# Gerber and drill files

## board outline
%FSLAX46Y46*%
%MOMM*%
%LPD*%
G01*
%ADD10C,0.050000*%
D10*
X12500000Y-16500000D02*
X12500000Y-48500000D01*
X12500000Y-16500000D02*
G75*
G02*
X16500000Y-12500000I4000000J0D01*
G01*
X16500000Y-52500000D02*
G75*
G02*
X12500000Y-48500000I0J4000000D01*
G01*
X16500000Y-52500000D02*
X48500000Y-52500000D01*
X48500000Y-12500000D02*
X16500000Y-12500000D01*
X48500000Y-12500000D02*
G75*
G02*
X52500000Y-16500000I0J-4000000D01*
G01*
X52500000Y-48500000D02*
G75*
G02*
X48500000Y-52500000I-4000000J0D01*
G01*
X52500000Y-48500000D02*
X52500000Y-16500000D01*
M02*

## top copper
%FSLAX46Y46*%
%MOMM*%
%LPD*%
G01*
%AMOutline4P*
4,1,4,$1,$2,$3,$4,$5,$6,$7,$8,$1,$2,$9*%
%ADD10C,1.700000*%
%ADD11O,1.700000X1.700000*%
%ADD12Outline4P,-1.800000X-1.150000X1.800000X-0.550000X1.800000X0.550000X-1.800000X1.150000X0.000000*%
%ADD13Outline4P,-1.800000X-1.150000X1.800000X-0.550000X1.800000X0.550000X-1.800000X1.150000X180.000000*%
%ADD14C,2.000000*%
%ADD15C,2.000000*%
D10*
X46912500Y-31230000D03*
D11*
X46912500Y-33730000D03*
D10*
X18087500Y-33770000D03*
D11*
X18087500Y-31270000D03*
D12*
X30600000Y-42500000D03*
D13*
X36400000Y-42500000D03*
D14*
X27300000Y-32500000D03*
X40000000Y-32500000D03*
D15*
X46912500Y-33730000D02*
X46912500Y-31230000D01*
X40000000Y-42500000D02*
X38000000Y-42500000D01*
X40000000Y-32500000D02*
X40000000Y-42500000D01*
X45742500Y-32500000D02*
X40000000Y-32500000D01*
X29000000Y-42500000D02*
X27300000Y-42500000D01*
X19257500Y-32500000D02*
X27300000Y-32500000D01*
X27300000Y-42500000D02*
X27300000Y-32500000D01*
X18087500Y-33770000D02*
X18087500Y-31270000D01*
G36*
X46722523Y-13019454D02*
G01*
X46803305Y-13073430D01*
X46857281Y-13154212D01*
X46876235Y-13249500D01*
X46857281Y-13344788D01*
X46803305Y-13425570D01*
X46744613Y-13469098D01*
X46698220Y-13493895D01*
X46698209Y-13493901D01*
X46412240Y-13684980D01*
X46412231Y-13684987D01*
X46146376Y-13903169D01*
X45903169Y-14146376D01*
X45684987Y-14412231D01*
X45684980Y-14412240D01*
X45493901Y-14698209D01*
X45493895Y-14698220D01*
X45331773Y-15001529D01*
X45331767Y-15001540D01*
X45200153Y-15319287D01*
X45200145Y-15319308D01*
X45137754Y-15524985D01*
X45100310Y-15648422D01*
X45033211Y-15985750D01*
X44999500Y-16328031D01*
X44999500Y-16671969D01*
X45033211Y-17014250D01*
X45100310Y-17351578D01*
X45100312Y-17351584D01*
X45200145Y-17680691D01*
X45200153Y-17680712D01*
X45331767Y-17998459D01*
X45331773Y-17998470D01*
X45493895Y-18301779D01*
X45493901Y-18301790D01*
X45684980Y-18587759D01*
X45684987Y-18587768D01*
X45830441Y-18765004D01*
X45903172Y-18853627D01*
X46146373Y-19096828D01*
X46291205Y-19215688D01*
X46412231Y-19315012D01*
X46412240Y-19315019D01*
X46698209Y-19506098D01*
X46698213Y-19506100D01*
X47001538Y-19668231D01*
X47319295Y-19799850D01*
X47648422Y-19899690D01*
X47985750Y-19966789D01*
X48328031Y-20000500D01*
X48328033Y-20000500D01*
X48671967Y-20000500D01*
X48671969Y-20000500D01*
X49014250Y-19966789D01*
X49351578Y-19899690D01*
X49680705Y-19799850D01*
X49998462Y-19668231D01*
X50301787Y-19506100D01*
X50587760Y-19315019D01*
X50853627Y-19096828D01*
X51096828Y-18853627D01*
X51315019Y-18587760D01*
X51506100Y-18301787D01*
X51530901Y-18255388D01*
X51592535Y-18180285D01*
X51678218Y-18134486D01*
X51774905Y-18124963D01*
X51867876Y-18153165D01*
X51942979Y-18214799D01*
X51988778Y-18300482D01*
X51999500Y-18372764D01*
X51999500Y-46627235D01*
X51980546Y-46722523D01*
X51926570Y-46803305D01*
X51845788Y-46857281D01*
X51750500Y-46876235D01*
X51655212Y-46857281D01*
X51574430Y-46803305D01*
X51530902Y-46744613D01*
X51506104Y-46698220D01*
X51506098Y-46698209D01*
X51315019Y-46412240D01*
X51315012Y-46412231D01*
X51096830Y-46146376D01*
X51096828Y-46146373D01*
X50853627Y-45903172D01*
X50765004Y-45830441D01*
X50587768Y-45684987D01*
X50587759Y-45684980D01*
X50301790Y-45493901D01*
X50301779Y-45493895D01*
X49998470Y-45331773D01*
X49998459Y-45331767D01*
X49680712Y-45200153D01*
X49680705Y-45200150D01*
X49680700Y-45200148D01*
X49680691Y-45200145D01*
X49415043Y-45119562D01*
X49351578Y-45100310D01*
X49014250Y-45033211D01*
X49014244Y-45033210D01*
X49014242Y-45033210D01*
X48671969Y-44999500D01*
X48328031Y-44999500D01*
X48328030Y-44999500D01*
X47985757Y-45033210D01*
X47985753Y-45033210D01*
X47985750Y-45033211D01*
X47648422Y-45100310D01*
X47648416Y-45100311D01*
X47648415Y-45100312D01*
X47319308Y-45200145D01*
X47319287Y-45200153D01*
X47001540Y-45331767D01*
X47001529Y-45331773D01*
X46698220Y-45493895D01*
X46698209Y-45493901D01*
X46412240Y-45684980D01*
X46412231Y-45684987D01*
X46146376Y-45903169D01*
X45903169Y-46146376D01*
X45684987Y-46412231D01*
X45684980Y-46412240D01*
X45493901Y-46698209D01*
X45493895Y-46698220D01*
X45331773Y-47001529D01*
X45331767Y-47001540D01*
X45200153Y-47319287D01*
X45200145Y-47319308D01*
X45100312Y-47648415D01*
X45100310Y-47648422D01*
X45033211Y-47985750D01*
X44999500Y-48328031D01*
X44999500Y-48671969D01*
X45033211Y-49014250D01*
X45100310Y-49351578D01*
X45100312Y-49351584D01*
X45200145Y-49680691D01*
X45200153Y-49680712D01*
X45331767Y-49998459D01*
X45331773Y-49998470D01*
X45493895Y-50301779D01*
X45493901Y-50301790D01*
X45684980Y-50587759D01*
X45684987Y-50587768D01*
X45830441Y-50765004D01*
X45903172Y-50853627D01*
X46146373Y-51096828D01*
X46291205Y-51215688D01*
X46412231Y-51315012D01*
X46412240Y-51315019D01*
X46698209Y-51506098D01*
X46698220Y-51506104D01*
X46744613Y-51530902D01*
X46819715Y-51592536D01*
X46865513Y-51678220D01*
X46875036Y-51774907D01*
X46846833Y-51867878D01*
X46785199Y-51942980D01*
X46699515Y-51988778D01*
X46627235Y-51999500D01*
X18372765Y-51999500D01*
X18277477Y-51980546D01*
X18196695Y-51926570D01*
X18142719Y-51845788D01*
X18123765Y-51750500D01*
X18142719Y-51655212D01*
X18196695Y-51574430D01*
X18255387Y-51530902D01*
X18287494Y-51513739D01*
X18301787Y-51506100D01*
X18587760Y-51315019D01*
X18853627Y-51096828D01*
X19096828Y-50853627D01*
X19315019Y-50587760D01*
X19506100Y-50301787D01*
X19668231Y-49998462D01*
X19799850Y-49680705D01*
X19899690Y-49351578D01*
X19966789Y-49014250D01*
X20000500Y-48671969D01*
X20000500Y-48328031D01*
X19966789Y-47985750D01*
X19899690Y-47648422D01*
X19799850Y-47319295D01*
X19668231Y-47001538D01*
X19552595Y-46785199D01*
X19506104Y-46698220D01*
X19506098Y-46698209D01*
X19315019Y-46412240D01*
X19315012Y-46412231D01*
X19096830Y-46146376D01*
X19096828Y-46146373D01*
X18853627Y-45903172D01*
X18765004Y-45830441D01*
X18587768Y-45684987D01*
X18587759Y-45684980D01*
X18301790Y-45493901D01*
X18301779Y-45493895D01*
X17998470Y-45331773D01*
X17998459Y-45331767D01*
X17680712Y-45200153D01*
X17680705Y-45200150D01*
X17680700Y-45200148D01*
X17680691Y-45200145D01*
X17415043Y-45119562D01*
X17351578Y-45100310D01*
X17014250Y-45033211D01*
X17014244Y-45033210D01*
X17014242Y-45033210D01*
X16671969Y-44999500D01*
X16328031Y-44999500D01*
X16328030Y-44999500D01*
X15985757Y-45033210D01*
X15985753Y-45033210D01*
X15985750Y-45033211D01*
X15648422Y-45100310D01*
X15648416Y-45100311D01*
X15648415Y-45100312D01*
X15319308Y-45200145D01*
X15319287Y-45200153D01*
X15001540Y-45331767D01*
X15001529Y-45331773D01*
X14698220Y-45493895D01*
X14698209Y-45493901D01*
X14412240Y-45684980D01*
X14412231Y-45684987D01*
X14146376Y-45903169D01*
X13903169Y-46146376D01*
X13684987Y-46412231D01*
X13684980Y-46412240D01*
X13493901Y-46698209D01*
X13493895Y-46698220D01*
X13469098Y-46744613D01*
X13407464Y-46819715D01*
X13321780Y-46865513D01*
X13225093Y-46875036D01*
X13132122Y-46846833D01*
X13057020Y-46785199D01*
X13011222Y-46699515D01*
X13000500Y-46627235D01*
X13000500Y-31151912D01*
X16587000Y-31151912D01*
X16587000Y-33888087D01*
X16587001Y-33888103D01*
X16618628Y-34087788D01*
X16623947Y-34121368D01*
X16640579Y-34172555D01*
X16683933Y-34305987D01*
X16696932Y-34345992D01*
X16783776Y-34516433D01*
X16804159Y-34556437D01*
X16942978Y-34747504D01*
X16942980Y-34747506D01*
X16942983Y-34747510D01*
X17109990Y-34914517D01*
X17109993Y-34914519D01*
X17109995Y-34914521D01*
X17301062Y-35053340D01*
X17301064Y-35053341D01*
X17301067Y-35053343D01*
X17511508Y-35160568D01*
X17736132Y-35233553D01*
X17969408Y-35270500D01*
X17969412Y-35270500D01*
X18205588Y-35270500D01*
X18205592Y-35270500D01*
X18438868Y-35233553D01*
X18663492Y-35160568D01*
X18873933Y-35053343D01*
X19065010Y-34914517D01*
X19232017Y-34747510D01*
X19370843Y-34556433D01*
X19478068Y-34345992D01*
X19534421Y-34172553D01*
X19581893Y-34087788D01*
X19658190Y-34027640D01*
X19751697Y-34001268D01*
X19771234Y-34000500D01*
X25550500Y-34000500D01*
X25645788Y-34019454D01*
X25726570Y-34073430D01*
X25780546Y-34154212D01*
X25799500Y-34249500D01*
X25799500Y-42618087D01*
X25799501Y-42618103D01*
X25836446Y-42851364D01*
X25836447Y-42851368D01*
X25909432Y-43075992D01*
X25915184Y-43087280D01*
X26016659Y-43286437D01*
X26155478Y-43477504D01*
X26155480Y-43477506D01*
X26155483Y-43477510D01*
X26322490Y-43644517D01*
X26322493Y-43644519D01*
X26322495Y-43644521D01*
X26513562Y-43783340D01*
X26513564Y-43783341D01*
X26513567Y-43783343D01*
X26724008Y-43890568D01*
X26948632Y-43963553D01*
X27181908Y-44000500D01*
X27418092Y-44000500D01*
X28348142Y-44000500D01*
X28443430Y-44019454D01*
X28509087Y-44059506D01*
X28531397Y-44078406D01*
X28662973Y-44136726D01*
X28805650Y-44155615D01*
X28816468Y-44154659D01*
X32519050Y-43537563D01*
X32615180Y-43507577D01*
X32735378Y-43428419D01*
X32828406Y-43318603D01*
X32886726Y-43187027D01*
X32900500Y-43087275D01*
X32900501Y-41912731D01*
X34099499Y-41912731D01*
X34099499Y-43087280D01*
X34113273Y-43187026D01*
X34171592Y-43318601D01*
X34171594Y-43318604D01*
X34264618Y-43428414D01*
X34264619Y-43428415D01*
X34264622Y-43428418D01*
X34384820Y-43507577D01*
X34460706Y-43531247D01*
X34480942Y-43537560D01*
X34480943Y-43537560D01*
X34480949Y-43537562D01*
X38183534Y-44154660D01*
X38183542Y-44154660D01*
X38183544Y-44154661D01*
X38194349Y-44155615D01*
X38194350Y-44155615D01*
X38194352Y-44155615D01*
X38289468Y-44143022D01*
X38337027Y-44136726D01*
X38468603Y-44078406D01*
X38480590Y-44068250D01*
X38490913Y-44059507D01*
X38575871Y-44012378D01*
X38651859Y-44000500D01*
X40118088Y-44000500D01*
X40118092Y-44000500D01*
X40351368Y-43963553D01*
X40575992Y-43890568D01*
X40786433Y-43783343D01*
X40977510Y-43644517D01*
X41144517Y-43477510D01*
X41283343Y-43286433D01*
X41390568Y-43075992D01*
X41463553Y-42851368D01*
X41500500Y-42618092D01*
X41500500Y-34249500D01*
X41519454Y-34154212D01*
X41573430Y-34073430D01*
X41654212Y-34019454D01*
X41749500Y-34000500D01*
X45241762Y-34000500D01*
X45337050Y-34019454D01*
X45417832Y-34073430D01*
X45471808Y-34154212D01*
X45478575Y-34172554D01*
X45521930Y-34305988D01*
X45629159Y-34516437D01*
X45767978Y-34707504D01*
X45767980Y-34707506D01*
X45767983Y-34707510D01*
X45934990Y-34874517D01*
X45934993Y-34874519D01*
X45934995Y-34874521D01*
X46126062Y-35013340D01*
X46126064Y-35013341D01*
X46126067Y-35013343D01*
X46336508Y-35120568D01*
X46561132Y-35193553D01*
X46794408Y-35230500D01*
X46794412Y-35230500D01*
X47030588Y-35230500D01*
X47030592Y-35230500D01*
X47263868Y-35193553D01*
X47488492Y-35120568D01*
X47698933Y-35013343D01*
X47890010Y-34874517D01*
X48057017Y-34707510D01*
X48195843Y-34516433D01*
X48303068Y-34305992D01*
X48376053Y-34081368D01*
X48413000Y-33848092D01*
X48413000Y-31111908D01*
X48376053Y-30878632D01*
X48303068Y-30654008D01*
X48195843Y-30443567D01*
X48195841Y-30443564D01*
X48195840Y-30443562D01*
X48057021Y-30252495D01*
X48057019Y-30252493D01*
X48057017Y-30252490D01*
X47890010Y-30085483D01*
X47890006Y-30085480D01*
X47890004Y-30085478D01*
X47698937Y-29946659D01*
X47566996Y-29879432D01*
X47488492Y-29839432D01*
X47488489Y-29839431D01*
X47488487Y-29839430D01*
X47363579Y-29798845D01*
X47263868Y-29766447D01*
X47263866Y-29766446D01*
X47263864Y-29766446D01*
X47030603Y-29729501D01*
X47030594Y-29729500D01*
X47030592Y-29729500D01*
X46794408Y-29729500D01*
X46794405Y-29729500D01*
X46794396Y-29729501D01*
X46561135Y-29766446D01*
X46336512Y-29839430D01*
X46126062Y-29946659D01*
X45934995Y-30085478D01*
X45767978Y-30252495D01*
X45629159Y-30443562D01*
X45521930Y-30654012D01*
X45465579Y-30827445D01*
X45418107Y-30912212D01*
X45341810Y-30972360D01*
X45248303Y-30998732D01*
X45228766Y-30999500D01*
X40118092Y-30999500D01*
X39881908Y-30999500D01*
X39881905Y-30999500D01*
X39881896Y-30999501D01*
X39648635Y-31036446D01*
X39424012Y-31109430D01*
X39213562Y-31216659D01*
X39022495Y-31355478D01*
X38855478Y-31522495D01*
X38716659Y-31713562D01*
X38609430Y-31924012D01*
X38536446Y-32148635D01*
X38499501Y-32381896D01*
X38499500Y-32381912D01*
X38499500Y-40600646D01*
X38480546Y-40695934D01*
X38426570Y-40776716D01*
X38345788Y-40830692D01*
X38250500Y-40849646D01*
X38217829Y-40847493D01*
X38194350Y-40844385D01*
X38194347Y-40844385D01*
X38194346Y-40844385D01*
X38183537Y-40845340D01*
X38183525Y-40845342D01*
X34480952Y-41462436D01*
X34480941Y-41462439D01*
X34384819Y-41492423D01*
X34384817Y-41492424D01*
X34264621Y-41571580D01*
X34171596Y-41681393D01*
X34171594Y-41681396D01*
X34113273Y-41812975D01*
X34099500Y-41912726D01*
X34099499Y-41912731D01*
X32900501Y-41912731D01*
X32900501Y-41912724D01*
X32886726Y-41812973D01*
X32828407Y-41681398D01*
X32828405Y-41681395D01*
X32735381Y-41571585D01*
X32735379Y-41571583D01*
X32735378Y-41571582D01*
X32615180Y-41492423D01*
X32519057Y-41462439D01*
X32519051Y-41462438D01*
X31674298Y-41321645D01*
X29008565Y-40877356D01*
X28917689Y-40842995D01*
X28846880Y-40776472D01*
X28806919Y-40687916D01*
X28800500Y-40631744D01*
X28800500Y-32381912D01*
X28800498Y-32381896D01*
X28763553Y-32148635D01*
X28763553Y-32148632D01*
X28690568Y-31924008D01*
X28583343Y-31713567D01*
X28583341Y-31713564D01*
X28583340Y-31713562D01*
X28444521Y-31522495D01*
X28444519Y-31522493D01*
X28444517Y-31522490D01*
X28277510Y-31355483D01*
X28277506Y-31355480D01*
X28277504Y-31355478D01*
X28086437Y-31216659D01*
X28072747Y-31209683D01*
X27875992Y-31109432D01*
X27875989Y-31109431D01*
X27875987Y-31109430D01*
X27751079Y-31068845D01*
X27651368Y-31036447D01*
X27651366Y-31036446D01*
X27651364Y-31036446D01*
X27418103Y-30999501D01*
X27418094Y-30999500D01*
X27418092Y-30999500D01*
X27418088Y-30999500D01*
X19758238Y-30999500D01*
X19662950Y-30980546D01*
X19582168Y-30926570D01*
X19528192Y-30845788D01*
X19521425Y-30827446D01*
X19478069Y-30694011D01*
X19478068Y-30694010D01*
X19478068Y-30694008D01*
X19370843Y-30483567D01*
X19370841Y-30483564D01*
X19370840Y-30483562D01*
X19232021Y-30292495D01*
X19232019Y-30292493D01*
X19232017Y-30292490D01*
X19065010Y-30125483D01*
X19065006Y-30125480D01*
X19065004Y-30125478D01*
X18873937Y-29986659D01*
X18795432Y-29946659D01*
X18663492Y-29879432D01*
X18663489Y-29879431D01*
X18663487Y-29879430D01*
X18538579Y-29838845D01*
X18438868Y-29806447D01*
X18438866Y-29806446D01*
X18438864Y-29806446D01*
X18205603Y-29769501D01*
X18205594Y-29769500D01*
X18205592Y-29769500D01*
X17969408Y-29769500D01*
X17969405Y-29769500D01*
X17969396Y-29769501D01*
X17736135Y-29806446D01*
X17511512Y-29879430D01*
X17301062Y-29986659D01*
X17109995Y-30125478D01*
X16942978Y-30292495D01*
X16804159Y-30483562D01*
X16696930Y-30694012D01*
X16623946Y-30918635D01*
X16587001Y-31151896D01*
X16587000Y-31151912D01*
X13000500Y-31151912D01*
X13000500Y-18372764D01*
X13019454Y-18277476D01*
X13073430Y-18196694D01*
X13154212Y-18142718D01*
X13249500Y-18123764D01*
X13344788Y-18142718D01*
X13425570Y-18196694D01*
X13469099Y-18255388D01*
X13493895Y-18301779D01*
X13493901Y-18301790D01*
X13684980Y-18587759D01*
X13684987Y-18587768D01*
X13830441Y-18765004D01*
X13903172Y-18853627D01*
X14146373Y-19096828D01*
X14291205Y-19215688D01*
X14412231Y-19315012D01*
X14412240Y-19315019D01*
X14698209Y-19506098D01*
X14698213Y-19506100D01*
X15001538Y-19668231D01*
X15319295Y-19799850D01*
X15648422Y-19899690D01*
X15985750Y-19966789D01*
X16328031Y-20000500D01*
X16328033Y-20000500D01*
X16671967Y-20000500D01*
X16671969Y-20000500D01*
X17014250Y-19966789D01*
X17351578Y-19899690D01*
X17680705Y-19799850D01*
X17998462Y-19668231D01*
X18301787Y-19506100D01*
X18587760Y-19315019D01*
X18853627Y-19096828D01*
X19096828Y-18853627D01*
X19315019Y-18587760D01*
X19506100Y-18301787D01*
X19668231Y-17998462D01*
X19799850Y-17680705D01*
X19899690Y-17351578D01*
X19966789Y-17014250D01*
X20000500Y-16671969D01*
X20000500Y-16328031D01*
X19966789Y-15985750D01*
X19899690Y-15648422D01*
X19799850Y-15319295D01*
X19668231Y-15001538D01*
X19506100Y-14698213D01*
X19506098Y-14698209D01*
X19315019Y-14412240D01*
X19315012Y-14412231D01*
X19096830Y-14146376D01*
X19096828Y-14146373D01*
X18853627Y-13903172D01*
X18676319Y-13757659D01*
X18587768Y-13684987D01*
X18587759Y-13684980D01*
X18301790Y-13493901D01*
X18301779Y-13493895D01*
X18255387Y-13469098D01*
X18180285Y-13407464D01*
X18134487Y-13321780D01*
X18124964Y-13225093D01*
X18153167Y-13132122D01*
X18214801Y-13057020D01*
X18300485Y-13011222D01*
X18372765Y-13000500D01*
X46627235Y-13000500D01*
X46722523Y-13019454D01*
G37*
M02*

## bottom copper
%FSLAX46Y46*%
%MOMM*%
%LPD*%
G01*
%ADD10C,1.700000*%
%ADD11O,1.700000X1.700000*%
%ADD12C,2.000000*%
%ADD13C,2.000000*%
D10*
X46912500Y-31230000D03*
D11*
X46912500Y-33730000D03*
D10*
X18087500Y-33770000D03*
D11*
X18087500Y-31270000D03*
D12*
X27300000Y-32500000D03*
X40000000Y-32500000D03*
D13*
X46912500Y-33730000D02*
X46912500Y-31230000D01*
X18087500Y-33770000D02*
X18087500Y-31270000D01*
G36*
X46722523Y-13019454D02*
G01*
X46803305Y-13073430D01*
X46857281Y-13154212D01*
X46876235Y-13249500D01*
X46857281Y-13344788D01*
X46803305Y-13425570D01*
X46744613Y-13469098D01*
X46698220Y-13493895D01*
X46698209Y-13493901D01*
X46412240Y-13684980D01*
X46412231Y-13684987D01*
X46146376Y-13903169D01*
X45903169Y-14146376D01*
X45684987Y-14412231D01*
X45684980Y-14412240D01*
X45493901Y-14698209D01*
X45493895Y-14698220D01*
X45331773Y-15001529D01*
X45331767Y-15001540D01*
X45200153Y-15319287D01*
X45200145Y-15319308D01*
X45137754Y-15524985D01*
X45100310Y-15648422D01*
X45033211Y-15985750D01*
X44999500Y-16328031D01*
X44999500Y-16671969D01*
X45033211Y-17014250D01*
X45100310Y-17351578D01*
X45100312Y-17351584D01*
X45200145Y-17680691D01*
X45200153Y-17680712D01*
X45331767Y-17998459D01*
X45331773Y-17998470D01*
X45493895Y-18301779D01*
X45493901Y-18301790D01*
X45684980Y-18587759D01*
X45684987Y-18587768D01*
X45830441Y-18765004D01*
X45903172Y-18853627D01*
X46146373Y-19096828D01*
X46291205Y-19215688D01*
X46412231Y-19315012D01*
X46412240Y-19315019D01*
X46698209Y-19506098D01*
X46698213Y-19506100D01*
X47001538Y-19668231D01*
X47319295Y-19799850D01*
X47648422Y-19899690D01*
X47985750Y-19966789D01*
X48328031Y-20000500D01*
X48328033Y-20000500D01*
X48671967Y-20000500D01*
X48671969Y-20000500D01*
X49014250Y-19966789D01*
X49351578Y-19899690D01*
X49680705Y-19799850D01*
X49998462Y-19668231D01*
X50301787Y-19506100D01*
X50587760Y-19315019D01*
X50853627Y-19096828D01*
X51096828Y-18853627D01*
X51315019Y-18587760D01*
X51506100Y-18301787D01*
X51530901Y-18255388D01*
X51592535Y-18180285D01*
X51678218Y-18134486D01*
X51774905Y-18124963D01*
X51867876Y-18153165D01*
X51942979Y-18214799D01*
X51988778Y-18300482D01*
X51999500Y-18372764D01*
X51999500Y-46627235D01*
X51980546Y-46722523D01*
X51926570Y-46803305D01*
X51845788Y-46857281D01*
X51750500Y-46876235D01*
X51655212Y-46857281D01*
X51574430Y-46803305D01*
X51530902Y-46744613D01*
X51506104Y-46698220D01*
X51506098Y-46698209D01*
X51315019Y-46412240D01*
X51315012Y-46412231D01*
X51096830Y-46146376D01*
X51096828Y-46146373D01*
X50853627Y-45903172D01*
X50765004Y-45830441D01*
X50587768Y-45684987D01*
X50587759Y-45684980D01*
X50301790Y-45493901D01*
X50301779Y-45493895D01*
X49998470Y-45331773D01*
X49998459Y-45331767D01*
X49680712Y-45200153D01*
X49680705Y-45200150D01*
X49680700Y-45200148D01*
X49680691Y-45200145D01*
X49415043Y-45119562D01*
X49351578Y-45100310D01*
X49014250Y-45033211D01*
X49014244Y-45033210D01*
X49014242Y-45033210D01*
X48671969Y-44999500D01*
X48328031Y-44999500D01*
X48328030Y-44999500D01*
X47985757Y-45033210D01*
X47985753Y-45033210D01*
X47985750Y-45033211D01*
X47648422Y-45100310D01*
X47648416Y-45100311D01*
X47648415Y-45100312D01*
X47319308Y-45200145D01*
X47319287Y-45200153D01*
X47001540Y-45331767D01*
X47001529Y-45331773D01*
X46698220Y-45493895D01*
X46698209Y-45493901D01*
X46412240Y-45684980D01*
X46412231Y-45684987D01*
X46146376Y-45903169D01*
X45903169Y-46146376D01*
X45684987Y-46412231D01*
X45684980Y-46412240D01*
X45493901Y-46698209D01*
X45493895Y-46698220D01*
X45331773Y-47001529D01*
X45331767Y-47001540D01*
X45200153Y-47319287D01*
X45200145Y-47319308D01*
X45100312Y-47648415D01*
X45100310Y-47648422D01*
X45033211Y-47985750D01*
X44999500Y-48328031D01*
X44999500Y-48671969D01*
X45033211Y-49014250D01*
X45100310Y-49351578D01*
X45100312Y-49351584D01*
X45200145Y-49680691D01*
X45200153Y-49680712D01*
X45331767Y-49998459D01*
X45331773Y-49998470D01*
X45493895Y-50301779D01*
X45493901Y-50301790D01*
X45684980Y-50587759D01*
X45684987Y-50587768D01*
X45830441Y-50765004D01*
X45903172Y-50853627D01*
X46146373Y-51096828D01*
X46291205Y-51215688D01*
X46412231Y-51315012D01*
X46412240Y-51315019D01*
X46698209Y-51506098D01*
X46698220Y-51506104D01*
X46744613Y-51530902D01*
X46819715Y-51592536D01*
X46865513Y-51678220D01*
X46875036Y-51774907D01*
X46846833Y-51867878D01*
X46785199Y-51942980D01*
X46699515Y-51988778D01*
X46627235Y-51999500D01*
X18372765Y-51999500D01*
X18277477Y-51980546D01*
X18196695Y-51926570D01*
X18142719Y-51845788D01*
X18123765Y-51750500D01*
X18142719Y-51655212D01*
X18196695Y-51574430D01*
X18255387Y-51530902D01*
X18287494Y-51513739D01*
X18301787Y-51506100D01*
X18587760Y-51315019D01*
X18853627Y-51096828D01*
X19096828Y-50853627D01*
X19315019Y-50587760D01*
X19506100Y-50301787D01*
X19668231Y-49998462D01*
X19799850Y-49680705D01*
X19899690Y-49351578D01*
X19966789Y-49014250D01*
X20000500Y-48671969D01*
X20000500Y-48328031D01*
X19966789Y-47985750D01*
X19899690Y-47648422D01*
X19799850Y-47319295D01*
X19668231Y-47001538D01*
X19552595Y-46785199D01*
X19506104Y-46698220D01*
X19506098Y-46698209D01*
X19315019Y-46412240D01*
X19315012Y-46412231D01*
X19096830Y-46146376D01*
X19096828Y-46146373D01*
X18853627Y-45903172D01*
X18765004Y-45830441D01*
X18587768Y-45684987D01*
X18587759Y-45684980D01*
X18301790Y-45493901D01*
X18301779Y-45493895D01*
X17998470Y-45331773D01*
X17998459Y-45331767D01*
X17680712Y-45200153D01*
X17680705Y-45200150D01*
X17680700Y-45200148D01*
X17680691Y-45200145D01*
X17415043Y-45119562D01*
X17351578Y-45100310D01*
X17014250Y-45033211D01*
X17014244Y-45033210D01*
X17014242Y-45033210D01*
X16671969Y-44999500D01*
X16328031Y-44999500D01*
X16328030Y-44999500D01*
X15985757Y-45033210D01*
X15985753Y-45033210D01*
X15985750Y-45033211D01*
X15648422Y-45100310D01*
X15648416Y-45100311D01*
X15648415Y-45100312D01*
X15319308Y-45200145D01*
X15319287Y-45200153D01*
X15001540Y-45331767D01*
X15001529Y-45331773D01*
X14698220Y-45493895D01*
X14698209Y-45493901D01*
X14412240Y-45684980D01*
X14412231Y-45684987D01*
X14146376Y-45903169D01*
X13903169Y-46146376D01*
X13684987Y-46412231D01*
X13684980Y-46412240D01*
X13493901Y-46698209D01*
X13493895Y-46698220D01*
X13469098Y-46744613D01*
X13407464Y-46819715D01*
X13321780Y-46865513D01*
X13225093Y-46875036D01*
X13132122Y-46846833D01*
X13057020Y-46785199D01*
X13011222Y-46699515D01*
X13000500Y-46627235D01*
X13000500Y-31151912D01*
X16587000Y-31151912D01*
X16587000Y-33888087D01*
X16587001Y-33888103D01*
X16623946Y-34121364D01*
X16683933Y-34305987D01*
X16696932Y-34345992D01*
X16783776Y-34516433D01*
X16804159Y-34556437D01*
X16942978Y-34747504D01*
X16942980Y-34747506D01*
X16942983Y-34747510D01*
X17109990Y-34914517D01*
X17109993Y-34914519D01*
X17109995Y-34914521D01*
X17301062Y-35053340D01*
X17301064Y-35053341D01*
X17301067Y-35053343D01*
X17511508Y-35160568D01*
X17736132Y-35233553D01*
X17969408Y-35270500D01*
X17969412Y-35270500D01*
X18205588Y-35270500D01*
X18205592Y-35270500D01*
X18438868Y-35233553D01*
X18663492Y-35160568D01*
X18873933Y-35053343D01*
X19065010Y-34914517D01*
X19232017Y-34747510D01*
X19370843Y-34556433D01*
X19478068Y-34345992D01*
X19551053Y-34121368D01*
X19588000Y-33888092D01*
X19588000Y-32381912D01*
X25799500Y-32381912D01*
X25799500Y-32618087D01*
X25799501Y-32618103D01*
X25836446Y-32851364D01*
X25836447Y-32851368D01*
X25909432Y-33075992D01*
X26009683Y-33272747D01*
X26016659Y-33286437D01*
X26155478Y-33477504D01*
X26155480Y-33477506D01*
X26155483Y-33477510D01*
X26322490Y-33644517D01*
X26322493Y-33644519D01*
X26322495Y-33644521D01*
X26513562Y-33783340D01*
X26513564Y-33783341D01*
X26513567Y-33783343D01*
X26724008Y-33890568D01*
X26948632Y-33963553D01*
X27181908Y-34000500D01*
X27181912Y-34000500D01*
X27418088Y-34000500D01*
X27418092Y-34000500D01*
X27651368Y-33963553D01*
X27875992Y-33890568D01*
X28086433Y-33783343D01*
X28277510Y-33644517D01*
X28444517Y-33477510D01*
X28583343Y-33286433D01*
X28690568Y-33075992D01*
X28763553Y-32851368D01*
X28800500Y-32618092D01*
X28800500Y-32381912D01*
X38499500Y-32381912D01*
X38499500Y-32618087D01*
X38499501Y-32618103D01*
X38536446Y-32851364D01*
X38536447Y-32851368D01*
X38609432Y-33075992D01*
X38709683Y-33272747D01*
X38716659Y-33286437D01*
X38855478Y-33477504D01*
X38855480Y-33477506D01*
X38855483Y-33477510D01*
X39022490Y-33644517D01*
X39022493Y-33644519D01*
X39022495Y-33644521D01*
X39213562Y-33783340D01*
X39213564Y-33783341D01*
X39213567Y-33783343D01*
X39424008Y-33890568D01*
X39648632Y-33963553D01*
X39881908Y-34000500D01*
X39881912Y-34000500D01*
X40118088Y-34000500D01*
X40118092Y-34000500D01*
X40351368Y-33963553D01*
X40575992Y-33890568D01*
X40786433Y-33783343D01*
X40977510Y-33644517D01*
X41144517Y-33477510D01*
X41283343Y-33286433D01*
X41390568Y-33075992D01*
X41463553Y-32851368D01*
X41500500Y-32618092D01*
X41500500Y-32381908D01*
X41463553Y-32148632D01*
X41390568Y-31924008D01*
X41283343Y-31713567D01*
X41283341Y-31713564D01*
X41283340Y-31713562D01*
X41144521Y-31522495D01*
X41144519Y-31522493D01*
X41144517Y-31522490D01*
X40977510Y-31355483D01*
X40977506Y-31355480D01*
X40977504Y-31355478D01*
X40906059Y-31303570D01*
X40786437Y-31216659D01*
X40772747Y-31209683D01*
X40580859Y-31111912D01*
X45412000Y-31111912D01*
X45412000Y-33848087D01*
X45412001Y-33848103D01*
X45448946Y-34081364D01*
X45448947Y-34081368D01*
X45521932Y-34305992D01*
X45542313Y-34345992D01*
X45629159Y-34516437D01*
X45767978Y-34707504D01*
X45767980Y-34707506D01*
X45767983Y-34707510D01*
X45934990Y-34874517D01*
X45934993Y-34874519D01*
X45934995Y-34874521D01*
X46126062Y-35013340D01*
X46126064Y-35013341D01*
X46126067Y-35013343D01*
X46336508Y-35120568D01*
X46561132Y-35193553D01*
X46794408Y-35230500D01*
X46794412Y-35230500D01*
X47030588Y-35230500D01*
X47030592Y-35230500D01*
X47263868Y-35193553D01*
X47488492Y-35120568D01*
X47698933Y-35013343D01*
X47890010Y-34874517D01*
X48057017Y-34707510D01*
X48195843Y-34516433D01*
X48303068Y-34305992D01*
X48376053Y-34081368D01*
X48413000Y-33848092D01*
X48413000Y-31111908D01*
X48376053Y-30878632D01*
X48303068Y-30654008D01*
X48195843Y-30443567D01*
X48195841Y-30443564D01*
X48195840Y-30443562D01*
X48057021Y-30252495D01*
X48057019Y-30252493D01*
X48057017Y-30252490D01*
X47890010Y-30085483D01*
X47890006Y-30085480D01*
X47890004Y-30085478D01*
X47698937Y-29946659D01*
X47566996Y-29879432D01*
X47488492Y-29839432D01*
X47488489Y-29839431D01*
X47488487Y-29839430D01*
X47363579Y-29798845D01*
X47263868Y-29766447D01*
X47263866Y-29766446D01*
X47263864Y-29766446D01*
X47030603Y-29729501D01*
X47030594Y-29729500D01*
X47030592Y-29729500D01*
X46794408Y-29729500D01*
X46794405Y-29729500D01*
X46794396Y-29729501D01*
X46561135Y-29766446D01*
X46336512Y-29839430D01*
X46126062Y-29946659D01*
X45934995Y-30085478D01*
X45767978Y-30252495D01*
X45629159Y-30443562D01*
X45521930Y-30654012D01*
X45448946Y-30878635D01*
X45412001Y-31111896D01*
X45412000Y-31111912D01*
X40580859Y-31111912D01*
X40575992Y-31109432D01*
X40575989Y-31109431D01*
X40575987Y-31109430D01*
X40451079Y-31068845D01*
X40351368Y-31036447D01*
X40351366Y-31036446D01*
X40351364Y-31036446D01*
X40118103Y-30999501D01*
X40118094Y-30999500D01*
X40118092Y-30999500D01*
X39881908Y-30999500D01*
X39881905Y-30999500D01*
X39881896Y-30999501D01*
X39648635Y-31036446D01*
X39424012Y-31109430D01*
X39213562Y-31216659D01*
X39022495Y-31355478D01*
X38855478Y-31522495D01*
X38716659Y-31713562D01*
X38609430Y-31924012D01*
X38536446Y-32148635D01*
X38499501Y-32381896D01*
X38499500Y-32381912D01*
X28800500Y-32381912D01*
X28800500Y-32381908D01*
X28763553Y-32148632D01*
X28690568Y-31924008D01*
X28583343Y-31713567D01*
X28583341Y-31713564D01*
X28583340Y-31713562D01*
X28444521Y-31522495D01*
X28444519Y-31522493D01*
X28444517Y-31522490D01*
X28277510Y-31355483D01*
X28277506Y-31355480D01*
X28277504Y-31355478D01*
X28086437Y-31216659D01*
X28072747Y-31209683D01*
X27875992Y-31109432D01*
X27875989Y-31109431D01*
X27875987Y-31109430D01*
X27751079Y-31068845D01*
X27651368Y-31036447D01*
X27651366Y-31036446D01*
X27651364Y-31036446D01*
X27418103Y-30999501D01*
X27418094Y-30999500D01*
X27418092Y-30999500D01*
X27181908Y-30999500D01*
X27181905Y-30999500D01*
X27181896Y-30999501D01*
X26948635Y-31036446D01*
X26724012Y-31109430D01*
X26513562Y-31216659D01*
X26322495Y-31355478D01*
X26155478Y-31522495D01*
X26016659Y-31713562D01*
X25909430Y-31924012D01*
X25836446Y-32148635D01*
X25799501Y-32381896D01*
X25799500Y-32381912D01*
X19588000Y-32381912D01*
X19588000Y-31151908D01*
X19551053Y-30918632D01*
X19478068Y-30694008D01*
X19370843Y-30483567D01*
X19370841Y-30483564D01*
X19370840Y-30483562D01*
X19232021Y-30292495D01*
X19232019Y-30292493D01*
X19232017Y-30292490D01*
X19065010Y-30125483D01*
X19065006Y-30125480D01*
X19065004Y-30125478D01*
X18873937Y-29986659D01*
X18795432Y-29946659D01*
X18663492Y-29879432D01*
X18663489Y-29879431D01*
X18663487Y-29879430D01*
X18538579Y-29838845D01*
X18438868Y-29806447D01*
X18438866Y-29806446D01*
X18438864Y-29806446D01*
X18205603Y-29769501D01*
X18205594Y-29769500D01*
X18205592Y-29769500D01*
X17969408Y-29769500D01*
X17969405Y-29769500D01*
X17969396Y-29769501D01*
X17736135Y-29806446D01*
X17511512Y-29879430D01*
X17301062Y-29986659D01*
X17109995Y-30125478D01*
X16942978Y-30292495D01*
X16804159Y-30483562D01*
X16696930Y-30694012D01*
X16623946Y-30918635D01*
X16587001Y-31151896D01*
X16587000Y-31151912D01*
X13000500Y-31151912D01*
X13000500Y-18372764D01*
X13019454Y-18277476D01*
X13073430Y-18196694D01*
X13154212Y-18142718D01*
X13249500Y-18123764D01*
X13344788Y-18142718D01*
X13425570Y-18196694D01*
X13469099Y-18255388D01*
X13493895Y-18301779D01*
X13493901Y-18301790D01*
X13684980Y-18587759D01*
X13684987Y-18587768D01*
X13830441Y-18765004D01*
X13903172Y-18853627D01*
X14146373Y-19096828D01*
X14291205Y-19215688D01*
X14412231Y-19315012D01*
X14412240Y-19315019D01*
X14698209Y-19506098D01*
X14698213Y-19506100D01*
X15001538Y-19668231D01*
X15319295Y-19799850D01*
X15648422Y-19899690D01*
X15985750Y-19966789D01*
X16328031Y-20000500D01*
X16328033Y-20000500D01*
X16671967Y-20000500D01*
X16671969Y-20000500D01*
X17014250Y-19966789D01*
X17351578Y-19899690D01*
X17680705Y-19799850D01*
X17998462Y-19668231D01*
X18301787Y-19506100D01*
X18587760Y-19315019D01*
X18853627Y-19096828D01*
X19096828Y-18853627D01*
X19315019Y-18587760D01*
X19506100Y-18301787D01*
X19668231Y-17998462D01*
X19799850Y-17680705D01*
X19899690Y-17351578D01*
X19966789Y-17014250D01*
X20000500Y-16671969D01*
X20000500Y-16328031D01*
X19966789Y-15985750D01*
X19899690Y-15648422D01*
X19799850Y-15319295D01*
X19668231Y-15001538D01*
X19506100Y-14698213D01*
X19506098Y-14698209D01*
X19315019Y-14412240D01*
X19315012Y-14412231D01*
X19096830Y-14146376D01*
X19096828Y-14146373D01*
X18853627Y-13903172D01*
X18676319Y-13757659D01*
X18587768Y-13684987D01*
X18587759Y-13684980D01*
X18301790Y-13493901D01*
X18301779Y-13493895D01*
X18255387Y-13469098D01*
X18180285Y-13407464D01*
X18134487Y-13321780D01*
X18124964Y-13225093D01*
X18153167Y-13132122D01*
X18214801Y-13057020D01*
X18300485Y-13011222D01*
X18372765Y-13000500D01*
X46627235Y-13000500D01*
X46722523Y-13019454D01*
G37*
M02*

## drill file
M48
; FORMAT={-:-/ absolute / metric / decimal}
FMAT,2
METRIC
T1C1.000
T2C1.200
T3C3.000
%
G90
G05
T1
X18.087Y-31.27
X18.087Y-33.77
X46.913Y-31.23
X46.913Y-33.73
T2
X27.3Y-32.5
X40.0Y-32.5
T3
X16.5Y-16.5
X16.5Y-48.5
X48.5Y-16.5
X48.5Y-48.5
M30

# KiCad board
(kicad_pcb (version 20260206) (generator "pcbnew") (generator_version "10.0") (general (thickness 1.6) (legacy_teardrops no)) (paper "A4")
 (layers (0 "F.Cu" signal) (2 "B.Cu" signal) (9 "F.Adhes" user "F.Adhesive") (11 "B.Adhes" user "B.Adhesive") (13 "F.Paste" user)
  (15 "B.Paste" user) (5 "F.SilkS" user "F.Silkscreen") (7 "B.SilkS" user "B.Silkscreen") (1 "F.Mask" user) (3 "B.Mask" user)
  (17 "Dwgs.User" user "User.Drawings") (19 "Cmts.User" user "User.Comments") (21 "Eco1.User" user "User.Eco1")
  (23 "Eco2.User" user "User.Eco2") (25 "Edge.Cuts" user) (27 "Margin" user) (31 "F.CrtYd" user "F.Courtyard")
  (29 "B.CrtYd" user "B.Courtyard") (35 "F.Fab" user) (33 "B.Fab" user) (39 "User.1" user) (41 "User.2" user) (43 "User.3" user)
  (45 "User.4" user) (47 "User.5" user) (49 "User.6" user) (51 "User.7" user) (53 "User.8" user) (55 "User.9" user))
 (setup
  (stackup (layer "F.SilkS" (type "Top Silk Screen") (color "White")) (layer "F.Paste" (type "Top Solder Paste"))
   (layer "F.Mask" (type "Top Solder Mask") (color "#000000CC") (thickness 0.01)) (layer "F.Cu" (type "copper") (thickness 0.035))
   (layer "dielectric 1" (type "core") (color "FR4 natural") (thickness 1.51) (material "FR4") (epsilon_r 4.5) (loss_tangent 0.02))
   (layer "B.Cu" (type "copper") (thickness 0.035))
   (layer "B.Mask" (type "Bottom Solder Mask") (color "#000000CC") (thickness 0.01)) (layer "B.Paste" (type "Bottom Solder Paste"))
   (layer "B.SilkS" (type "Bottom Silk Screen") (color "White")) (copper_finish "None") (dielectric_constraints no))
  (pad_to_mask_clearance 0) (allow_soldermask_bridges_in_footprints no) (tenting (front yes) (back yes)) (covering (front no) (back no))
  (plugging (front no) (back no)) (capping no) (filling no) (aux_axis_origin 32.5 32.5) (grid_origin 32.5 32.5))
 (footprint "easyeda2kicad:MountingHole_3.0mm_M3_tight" (layer "F.Cu") (at 16.5 16.5 90)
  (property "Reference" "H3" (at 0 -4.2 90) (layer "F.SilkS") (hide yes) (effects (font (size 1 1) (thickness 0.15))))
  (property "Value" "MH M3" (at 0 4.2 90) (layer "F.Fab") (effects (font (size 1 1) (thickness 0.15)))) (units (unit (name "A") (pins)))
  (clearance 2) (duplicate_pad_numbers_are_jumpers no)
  (pad "" np_thru_hole circle (at 0 0 90) (size 3 3) (drill 3) (layers "*.Cu" "*.Mask")))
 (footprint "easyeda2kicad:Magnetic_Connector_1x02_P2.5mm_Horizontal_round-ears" (layer "F.Cu") (at 47.0125 32.5)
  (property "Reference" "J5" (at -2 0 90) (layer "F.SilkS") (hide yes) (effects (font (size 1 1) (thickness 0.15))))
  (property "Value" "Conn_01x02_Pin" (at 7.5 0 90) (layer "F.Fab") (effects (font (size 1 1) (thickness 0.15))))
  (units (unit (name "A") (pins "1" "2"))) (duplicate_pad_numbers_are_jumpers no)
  (pad "1" thru_hole circle (at -0.1 -1.27) (size 1.7 1.7) (drill 1) (layers "*.Cu" "*.Mask") (remove_unused_layers no) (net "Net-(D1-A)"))
  (pad "2" thru_hole oval (at -0.1 1.23) (size 1.7 1.7) (drill 1) (layers "*.Cu" "*.Mask") (remove_unused_layers no) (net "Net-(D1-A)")))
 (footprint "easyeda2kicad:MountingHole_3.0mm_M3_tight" (layer "F.Cu") (at 16.5 48.5 90)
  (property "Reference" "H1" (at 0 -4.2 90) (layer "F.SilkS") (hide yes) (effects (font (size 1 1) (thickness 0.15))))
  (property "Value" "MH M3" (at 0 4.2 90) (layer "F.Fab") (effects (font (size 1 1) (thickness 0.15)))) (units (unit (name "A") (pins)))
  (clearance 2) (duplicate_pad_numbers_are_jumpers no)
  (pad "" np_thru_hole circle (at 0 0 90) (size 3 3) (drill 3) (layers "*.Cu" "*.Mask")))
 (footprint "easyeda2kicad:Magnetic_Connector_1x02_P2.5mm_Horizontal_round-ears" (layer "F.Cu") (at 17.9875 32.5 180)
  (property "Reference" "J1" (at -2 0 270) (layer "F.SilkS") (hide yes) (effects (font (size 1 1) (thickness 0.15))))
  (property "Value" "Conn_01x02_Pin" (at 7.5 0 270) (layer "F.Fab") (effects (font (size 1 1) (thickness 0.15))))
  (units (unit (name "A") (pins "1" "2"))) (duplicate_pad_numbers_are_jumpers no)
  (pad "1" thru_hole circle (at -0.1 -1.27 180) (size 1.7 1.7) (drill 1) (layers "*.Cu" "*.Mask") (remove_unused_layers no)
   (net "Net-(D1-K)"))
  (pad "2" thru_hole oval (at -0.1 1.23 180) (size 1.7 1.7) (drill 1) (layers "*.Cu" "*.Mask") (remove_unused_layers no) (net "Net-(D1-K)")))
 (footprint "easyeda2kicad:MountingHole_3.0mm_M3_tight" (layer "F.Cu") (at 48.5 48.5 90)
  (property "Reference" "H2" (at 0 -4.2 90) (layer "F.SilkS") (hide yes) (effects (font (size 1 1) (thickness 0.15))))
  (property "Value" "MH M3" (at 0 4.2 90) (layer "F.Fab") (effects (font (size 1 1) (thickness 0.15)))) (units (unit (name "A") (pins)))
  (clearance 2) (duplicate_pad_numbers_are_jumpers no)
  (pad "" np_thru_hole circle (at 0 0 90) (size 3 3) (drill 3) (layers "*.Cu" "*.Mask")))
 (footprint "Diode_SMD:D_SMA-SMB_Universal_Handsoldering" (layer "F.Cu") (at 33.5 42.5)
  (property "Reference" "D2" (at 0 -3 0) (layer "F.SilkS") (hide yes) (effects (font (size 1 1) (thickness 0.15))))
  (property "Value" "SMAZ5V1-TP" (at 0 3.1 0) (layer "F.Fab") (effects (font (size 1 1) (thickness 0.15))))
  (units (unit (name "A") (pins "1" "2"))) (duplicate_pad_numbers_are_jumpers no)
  (pad "1" smd trapezoid (at -2.9 0) (size 3.6 1.7) (rect_delta 0.6 0) (layers "F.Cu" "F.Mask" "F.Paste") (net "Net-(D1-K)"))
  (pad "2" smd trapezoid (at 2.9 0 180) (size 3.6 1.7) (rect_delta 0.6 0) (layers "F.Cu" "F.Mask" "F.Paste") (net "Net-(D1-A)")))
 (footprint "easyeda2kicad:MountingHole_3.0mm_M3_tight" (layer "F.Cu") (at 48.5 16.5 90)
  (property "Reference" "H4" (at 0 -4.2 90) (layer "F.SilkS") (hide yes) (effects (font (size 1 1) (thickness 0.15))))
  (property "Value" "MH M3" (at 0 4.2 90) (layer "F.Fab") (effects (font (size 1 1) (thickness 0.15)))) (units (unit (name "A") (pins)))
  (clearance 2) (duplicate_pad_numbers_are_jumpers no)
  (pad "" np_thru_hole circle (at 0 0 90) (size 3 3) (drill 3) (layers "*.Cu" "*.Mask")))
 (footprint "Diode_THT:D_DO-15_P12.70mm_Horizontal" (layer "F.Cu") (at 27.3 32.5)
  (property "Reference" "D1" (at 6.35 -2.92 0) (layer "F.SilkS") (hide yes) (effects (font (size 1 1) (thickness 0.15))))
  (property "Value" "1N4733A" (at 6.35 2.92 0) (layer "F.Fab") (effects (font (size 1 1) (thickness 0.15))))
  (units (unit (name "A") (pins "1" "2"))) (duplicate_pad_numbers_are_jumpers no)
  (pad "1" thru_hole circle (at 0 0) (size 2 2) (drill 1.2) (layers "*.Cu" "*.Mask") (remove_unused_layers no) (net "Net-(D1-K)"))
  (pad "2" thru_hole circle (at 12.7 0) (size 2 2) (drill 1.2) (layers "*.Cu" "*.Mask") (remove_unused_layers no) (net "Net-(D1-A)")))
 (gr_line (start 12.5 16.5) (end 12.5 48.5) (stroke (width 0.05) (type default)) (layer "Edge.Cuts"))
 (gr_arc (start 12.5 16.5) (mid 13.671573 13.671573) (end 16.5 12.5) (stroke (width 0.05) (type default)) (layer "Edge.Cuts"))
 (gr_arc (start 16.5 52.5) (mid 13.671573 51.328427) (end 12.5 48.5) (stroke (width 0.05) (type default)) (layer "Edge.Cuts"))
 (gr_line (start 16.5 52.5) (end 48.5 52.5) (stroke (width 0.05) (type default)) (layer "Edge.Cuts"))
 (gr_line (start 48.5 12.5) (end 16.5 12.5) (stroke (width 0.05) (type default)) (layer "Edge.Cuts"))
 (gr_arc (start 48.5 12.5) (mid 51.328427 13.671573) (end 52.5 16.5) (stroke (width 0.05) (type default)) (layer "Edge.Cuts"))
 (gr_arc (start 52.5 48.5) (mid 51.328427 51.328427) (end 48.5 52.5) (stroke (width 0.05) (type default)) (layer "Edge.Cuts"))
 (gr_line (start 52.5 48.5) (end 52.5 16.5) (stroke (width 0.05) (type default)) (layer "Edge.Cuts"))
 (segment (start 46.9125 33.73) (end 46.9125 31.23) (width 2) (layer "F.Cu") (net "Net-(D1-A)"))
 (segment (start 40 42.5) (end 38 42.5) (width 2) (layer "F.Cu") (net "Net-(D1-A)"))
 (segment (start 40 32.5) (end 40 42.5) (width 2) (layer "F.Cu") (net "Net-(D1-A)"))
 (segment (start 45.7425 32.5) (end 40 32.5) (width 2) (layer "F.Cu") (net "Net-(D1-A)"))
 (segment (start 46.9125 33.73) (end 46.9125 31.23) (width 2) (layer "B.Cu") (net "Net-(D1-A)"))
 (segment (start 29 42.5) (end 27.3 42.5) (width 2) (layer "F.Cu") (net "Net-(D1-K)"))
 (segment (start 19.2575 32.5) (end 27.3 32.5) (width 2) (layer "F.Cu") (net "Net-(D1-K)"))
 (segment (start 27.3 42.5) (end 27.3 32.5) (width 2) (layer "F.Cu") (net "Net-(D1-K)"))
 (segment (start 18.0875 33.77) (end 18.0875 31.27) (width 2) (layer "F.Cu") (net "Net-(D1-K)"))
 (segment (start 18.0875 33.77) (end 18.0875 31.27) (width 2) (layer "B.Cu") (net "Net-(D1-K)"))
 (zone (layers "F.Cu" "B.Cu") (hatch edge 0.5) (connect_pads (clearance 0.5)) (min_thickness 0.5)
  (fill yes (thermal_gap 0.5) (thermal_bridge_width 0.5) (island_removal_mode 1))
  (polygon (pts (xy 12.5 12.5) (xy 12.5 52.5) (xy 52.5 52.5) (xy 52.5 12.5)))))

